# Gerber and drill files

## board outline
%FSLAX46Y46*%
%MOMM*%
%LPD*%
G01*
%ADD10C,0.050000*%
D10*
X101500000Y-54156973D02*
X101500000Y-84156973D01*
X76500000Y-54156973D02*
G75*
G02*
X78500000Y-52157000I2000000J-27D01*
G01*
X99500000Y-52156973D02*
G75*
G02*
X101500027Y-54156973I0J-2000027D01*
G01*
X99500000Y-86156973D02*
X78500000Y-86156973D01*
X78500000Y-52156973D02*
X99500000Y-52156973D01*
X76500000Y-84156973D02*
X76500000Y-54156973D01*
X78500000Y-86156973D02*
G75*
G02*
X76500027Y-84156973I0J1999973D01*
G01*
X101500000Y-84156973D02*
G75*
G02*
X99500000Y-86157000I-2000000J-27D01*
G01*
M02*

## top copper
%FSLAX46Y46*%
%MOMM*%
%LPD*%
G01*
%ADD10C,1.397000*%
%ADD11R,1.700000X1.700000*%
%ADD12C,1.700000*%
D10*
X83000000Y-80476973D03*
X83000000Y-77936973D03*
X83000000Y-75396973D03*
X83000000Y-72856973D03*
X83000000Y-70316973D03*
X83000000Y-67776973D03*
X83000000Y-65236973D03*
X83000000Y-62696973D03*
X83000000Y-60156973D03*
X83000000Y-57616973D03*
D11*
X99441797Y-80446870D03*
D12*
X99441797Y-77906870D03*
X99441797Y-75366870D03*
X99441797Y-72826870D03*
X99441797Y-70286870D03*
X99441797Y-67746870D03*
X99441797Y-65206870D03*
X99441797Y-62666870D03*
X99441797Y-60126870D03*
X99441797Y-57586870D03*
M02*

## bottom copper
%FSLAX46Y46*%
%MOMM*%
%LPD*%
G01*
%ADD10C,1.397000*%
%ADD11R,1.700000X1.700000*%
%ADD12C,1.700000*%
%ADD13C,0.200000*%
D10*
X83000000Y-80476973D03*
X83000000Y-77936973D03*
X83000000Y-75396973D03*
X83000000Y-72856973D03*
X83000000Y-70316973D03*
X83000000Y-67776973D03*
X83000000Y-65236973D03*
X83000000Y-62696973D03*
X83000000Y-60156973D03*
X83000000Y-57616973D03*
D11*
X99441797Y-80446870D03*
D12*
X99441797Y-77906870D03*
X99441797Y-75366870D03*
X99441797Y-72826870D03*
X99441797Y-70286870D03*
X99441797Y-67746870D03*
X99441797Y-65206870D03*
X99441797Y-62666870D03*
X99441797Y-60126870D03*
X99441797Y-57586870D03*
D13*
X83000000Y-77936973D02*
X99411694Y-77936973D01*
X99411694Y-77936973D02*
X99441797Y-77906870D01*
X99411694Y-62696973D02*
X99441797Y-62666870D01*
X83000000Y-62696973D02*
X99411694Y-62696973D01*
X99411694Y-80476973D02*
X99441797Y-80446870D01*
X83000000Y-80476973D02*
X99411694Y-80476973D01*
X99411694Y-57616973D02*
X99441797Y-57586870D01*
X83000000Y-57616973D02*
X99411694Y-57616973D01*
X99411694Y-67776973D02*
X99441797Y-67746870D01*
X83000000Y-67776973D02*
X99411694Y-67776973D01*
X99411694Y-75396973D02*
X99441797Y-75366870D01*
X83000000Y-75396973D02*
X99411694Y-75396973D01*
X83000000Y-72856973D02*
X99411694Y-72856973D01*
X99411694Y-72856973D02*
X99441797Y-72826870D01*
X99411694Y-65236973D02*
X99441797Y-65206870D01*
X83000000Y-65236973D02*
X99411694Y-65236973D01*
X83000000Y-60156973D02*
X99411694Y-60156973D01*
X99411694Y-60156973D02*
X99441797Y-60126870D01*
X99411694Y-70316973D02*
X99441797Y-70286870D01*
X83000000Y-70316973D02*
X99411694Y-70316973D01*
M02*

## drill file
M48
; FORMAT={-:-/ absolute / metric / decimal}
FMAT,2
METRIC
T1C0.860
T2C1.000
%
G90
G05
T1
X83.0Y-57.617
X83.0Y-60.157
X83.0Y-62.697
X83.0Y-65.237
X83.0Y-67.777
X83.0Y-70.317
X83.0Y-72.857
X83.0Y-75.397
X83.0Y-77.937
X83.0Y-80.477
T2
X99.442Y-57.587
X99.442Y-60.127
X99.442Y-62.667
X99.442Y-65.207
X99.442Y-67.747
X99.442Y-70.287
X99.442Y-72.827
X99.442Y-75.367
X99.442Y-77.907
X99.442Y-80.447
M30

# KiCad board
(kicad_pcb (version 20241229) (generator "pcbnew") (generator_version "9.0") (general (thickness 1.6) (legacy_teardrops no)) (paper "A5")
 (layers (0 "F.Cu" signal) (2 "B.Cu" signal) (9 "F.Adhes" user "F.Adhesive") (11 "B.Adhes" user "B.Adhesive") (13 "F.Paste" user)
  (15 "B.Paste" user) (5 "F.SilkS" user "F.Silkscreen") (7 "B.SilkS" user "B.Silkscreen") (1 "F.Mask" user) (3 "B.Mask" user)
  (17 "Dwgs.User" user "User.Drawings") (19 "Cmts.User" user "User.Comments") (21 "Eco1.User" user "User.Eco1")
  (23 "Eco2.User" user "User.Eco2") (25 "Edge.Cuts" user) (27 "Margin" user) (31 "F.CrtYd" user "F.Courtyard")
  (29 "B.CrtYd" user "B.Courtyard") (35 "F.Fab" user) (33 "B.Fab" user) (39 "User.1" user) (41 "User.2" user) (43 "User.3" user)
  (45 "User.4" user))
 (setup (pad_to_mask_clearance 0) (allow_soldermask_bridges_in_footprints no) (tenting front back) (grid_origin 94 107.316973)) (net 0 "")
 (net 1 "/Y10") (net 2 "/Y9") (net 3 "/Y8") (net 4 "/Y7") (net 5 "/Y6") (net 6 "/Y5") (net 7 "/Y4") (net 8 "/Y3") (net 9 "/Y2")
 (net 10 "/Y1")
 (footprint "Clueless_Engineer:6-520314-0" (layer "F.Cu") (at 83 69.046973 -90)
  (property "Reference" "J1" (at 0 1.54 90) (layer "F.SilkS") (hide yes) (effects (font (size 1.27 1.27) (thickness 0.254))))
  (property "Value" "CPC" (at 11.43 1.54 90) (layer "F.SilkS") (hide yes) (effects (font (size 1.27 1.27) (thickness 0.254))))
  (pad "1" thru_hole circle (at 11.43 0 270) (size 1.397 1.397) (drill 0.86) (layers "*.Cu" "*.Mask") (remove_unused_layers no)
   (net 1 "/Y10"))
  (pad "2" thru_hole circle (at 8.89 0 270) (size 1.397 1.397) (drill 0.86) (layers "*.Cu" "*.Mask") (remove_unused_layers no) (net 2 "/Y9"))
  (pad "3" thru_hole circle (at 6.35 0 270) (size 1.397 1.397) (drill 0.86) (layers "*.Cu" "*.Mask") (remove_unused_layers no) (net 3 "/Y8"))
  (pad "4" thru_hole circle (at 3.81 0 270) (size 1.397 1.397) (drill 0.86) (layers "*.Cu" "*.Mask") (remove_unused_layers no) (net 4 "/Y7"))
  (pad "5" thru_hole circle (at 1.27 0 270) (size 1.397 1.397) (drill 0.86) (layers "*.Cu" "*.Mask") (remove_unused_layers no) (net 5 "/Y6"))
  (pad "6" thru_hole circle (at -1.27 0 270) (size 1.397 1.397) (drill 0.86) (layers "*.Cu" "*.Mask") (remove_unused_layers no)
   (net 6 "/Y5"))
  (pad "7" thru_hole circle (at -3.81 0 270) (size 1.397 1.397) (drill 0.86) (layers "*.Cu" "*.Mask") (remove_unused_layers no)
   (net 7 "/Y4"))
  (pad "8" thru_hole circle (at -6.35 0 270) (size 1.397 1.397) (drill 0.86) (layers "*.Cu" "*.Mask") (remove_unused_layers no)
   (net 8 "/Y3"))
  (pad "9" thru_hole circle (at -8.89 0 270) (size 1.397 1.397) (drill 0.86) (layers "*.Cu" "*.Mask") (remove_unused_layers no)
   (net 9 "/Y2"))
  (pad "10" thru_hole circle (at -11.43 0 270) (size 1.397 1.397) (drill 0.86) (layers "*.Cu" "*.Mask") (remove_unused_layers no)
   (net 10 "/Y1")))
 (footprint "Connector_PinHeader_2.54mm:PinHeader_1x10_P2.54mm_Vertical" (layer "F.Cu") (at 99.441797 57.58687)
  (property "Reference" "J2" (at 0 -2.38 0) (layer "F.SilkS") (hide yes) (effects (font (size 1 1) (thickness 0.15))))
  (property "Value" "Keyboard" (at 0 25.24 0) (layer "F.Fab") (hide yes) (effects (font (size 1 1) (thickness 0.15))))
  (pad "1" thru_hole rect (at 0 22.86) (size 1.7 1.7) (drill 1) (layers "*.Cu" "*.Mask") (remove_unused_layers no) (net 1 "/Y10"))
  (pad "2" thru_hole circle (at 0 20.32) (size 1.7 1.7) (drill 1) (layers "*.Cu" "*.Mask") (remove_unused_layers no) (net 2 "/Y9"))
  (pad "3" thru_hole circle (at 0 17.78) (size 1.7 1.7) (drill 1) (layers "*.Cu" "*.Mask") (remove_unused_layers no) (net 3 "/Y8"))
  (pad "4" thru_hole circle (at 0 15.24) (size 1.7 1.7) (drill 1) (layers "*.Cu" "*.Mask") (remove_unused_layers no) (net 4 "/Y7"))
  (pad "5" thru_hole circle (at 0 12.7) (size 1.7 1.7) (drill 1) (layers "*.Cu" "*.Mask") (remove_unused_layers no) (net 5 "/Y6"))
  (pad "6" thru_hole circle (at 0 10.16) (size 1.7 1.7) (drill 1) (layers "*.Cu" "*.Mask") (remove_unused_layers no) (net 6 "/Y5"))
  (pad "7" thru_hole circle (at 0 7.62) (size 1.7 1.7) (drill 1) (layers "*.Cu" "*.Mask") (remove_unused_layers no) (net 7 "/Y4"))
  (pad "8" thru_hole circle (at 0 5.08) (size 1.7 1.7) (drill 1) (layers "*.Cu" "*.Mask") (remove_unused_layers no) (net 8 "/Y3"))
  (pad "9" thru_hole circle (at 0 2.54) (size 1.7 1.7) (drill 1) (layers "*.Cu" "*.Mask") (remove_unused_layers no) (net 9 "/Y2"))
  (pad "10" thru_hole circle (at 0 0) (size 1.7 1.7) (drill 1) (layers "*.Cu" "*.Mask") (remove_unused_layers no) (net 10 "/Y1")))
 (gr_line (start 101.5 54.156973) (end 101.5 84.156973) (stroke (width 0.05) (type default)) (layer "Edge.Cuts"))
 (gr_arc (start 76.5 54.156973) (mid 77.085786 52.742759) (end 78.5 52.156973) (stroke (width 0.05) (type default)) (layer "Edge.Cuts"))
 (gr_arc (start 99.5 52.156973) (mid 100.914214 52.742759) (end 101.5 54.156973) (stroke (width 0.05) (type default)) (layer "Edge.Cuts"))
 (gr_line (start 99.5 86.156973) (end 78.5 86.156973) (stroke (width 0.05) (type default)) (layer "Edge.Cuts"))
 (gr_line (start 78.5 52.156973) (end 99.5 52.156973) (stroke (width 0.05) (type default)) (layer "Edge.Cuts"))
 (gr_line (start 76.5 84.156973) (end 76.5 54.156973) (stroke (width 0.05) (type default)) (layer "Edge.Cuts"))
 (gr_arc (start 78.5 86.156973) (mid 77.085786 85.571187) (end 76.5 84.156973) (stroke (width 0.05) (type default)) (layer "Edge.Cuts"))
 (gr_arc (start 101.5 84.156973) (mid 100.914214 85.571187) (end 99.5 86.156973) (stroke (width 0.05) (type default)) (layer "Edge.Cuts"))
 (segment (start 83 77.936973) (end 99.411694 77.936973) (width 0.2) (layer "B.Cu") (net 2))
 (segment (start 99.411694 77.936973) (end 99.441797 77.90687) (width 0.2) (layer "B.Cu") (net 2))
 (segment (start 99.411694 62.696973) (end 99.441797 62.66687) (width 0.2) (layer "B.Cu") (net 8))
 (segment (start 83 62.696973) (end 99.411694 62.696973) (width 0.2) (layer "B.Cu") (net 8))
 (segment (start 99.411694 80.476973) (end 99.441797 80.44687) (width 0.2) (layer "B.Cu") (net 1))
 (segment (start 83 80.476973) (end 99.411694 80.476973) (width 0.2) (layer "B.Cu") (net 1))
 (segment (start 99.411694 57.616973) (end 99.441797 57.58687) (width 0.2) (layer "B.Cu") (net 10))
 (segment (start 83 57.616973) (end 99.411694 57.616973) (width 0.2) (layer "B.Cu") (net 10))
 (segment (start 99.411694 67.776973) (end 99.441797 67.74687) (width 0.2) (layer "B.Cu") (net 6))
 (segment (start 83 67.776973) (end 99.411694 67.776973) (width 0.2) (layer "B.Cu") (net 6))
 (segment (start 99.411694 75.396973) (end 99.441797 75.36687) (width 0.2) (layer "B.Cu") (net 3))
 (segment (start 83 75.396973) (end 99.411694 75.396973) (width 0.2) (layer "B.Cu") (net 3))
 (segment (start 83 72.856973) (end 99.411694 72.856973) (width 0.2) (layer "B.Cu") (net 4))
 (segment (start 99.411694 72.856973) (end 99.441797 72.82687) (width 0.2) (layer "B.Cu") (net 4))
 (segment (start 99.411694 65.236973) (end 99.441797 65.20687) (width 0.2) (layer "B.Cu") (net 7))
 (segment (start 83 65.236973) (end 99.411694 65.236973) (width 0.2) (layer "B.Cu") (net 7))
 (segment (start 83 60.156973) (end 99.411694 60.156973) (width 0.2) (layer "B.Cu") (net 9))
 (segment (start 99.411694 60.156973) (end 99.441797 60.12687) (width 0.2) (layer "B.Cu") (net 9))
 (segment (start 99.411694 70.316973) (end 99.441797 70.28687) (width 0.2) (layer "B.Cu") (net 5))
 (segment (start 83 70.316973) (end 99.411694 70.316973) (width 0.2) (layer "B.Cu") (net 5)))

